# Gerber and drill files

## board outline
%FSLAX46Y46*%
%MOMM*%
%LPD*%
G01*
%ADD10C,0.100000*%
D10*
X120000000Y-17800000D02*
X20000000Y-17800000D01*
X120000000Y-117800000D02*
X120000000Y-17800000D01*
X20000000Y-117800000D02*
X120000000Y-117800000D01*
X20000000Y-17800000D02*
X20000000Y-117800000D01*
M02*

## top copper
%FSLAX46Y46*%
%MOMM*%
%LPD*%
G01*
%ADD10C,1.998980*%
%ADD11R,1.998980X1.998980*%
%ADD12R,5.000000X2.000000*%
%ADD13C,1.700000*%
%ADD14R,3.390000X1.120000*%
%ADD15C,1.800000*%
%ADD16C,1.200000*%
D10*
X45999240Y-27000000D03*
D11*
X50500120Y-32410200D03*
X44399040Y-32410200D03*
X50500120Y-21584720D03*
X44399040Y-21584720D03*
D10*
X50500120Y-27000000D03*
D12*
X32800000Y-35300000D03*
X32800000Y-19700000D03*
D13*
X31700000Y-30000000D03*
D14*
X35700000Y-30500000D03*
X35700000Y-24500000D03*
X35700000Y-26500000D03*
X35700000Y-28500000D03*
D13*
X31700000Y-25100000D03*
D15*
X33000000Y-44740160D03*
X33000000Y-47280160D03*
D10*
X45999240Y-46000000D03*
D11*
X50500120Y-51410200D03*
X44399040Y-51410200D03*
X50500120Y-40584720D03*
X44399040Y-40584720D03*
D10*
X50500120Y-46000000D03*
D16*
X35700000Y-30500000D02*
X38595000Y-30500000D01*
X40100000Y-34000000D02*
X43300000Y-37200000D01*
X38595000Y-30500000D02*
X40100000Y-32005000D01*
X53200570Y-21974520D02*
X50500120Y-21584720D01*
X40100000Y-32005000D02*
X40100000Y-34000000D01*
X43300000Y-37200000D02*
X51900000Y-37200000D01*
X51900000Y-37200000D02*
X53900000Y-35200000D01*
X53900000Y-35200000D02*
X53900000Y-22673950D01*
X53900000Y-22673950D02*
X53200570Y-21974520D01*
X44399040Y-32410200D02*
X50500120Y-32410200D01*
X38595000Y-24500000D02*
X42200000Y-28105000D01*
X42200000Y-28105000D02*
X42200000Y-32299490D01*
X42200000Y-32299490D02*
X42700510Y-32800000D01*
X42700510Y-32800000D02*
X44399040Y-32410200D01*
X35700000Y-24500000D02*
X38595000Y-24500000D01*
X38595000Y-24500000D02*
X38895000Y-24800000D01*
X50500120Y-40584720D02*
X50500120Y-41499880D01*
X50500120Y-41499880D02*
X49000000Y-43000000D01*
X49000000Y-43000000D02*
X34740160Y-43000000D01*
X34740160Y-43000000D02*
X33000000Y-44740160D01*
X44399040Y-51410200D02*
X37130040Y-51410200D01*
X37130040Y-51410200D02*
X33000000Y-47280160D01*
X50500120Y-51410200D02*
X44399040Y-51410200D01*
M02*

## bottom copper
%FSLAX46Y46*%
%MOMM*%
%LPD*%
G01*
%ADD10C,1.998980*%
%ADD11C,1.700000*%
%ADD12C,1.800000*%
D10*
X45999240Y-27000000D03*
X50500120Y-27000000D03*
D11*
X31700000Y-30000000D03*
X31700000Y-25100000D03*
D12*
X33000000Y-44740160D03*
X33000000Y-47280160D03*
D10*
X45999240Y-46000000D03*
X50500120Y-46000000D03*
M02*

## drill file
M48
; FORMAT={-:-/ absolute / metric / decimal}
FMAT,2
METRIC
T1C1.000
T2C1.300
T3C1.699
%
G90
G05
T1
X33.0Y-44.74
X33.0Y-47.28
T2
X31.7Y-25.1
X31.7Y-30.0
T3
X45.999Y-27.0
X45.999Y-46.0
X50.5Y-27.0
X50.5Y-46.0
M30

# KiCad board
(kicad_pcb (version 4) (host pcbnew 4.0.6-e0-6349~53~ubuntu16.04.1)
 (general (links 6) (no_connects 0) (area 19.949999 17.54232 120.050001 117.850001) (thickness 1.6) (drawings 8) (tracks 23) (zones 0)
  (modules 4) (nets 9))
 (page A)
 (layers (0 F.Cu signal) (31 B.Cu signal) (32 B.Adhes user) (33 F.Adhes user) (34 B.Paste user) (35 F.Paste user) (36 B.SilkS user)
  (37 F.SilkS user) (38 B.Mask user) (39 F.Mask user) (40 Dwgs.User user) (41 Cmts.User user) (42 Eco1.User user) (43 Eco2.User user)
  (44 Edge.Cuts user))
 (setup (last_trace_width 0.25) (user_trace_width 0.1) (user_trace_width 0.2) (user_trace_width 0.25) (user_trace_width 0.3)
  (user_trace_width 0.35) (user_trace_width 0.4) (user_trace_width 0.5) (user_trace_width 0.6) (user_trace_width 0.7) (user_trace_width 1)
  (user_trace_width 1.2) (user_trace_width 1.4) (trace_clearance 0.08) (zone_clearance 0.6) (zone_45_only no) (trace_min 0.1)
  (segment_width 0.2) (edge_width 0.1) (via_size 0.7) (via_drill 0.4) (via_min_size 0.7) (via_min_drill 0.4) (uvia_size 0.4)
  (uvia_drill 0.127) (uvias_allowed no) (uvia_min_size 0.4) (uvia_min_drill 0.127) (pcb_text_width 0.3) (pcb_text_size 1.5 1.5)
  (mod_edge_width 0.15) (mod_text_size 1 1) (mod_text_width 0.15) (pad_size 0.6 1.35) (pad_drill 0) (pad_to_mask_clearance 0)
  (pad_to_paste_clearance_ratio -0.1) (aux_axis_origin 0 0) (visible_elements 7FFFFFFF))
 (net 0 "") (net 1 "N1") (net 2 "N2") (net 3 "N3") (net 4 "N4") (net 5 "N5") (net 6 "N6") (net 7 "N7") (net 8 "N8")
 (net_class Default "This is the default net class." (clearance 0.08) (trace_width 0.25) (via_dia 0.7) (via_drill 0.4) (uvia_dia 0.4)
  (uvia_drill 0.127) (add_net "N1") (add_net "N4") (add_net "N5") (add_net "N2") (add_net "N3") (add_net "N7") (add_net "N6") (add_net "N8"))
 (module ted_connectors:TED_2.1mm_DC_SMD (layer F.Cu) (at 47 27)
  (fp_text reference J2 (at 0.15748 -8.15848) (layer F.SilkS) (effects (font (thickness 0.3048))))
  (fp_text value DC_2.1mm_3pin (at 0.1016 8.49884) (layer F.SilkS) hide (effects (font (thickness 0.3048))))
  (pad "" np_thru_hole circle (at -1.00076 0) (size 1.99898 1.99898) (drill 1.69926) (layers *.Cu *.Mask F.SilkS))
  (pad 1 smd rect (at 3.50012 5.4102) (size 1.99898 1.99898) (layers F.Cu F.Paste F.Mask) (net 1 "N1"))
  (pad 1 smd rect (at -2.60096 5.4102) (size 1.99898 1.99898) (layers F.Cu F.Paste F.Mask) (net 1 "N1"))
  (pad 2 smd rect (at 3.50012 -5.41528) (size 1.99898 1.99898) (layers F.Cu F.Paste F.Mask) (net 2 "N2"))
  (pad 3 smd rect (at -2.60096 -5.41528) (size 1.99898 1.99898) (layers F.Cu F.Paste F.Mask) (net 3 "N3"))
  (pad "" np_thru_hole circle (at 3.50012 0) (size 1.99898 1.99898) (drill 1.69926) (layers *.Cu *.Mask F.SilkS)))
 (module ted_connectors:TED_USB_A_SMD (layer F.Cu) (at 28.2 27.5 270)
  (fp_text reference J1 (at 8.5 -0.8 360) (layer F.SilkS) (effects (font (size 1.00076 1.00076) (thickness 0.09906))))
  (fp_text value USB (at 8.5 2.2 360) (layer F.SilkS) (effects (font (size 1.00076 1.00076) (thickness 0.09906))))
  (pad GP smd rect (at 7.8 -4.6 270) (size 2 5) (layers F.Cu F.Paste F.Mask))
  (pad GP smd rect (at -7.8 -4.6 270) (size 2 5) (layers F.Cu F.Paste F.Mask))
  (pad "" np_thru_hole circle (at 2.5 -3.5 270) (size 1.7 1.7) (drill 1.3) (layers *.Cu *.Mask F.SilkS))
  (pad 4 smd rect (at 3 -7.5 270) (size 1.12 3.39) (layers F.Cu F.Paste F.Mask) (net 2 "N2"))
  (pad 1 smd rect (at -3 -7.5 270) (size 1.12 3.39) (layers F.Cu F.Paste F.Mask) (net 1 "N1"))
  (pad 2 smd rect (at -1 -7.5 270) (size 1.12 3.39) (layers F.Cu F.Paste F.Mask) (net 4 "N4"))
  (pad 3 smd rect (at 1 -7.5 270) (size 1.12 3.39) (layers F.Cu F.Paste F.Mask) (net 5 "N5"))
  (pad "" np_thru_hole circle (at -2.4 -3.5 270) (size 1.7 1.7) (drill 1.3) (layers *.Cu *.Mask F.SilkS)))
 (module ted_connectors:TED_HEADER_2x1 (layer F.Cu) (at 33 46 90)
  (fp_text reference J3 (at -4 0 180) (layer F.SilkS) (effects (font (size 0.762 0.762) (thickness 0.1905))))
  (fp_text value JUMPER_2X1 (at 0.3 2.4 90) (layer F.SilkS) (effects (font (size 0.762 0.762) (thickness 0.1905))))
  (pad 2 thru_hole circle (at 1.25984 0 90) (size 1.8 1.8) (drill 1) (layers *.Cu *.Mask F.SilkS) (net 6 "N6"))
  (pad 1 thru_hole circle (at -1.28016 0 90) (size 1.8 1.8) (drill 1) (layers *.Cu *.Mask F.SilkS) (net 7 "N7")))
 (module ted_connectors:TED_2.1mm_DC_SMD (layer F.Cu) (at 47 46)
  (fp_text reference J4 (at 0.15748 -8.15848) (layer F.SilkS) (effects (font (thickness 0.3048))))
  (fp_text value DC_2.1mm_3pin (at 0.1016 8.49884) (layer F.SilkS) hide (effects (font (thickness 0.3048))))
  (pad "" np_thru_hole circle (at -1.00076 0) (size 1.99898 1.99898) (drill 1.69926) (layers *.Cu *.Mask F.SilkS))
  (pad 1 smd rect (at 3.50012 5.4102) (size 1.99898 1.99898) (layers F.Cu F.Paste F.Mask) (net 7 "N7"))
  (pad 1 smd rect (at -2.60096 5.4102) (size 1.99898 1.99898) (layers F.Cu F.Paste F.Mask) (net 7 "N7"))
  (pad 2 smd rect (at 3.50012 -5.41528) (size 1.99898 1.99898) (layers F.Cu F.Paste F.Mask) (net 6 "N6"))
  (pad 3 smd rect (at -2.60096 -5.41528) (size 1.99898 1.99898) (layers F.Cu F.Paste F.Mask) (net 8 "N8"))
  (pad "" np_thru_hole circle (at 3.50012 0) (size 1.99898 1.99898) (drill 1.69926) (layers *.Cu *.Mask F.SilkS)))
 (gr_line (start 120 17.8) (end 20 17.8) (angle 90) (layer Edge.Cuts) (width 0.1))
 (gr_line (start 120 117.8) (end 120 17.8) (angle 90) (layer Edge.Cuts) (width 0.1))
 (gr_line (start 20 117.8) (end 120 117.8) (angle 90) (layer Edge.Cuts) (width 0.1))
 (gr_line (start 20 17.8) (end 20 117.8) (angle 90) (layer Edge.Cuts) (width 0.1))
 (segment (start 35.7 30.5) (end 38.595 30.5) (width 1.2) (layer F.Cu) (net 2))
 (segment (start 40.1 34) (end 43.3 37.2) (width 1.2) (layer F.Cu) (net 2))
 (segment (start 38.595 30.5) (end 40.1 32.005) (width 1.2) (layer F.Cu) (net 2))
 (segment (start 53.20057 21.97452) (end 50.50012 21.58472) (width 1.2) (layer F.Cu) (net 2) (status 20))
 (segment (start 40.1 32.005) (end 40.1 34) (width 1.2) (layer F.Cu) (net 2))
 (segment (start 43.3 37.2) (end 51.9 37.2) (width 1.2) (layer F.Cu) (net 2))
 (segment (start 51.9 37.2) (end 53.9 35.2) (width 1.2) (layer F.Cu) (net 2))
 (segment (start 53.9 35.2) (end 53.9 22.67395) (width 1.2) (layer F.Cu) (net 2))
 (segment (start 53.9 22.67395) (end 53.20057 21.97452) (width 1.2) (layer F.Cu) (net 2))
 (segment (start 44.39904 32.4102) (end 50.50012 32.4102) (width 1.2) (layer F.Cu) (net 1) (status 30))
 (segment (start 38.595 24.5) (end 42.2 28.105) (width 1.2) (layer F.Cu) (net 1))
 (segment (start 42.2 28.105) (end 42.2 32.29949) (width 1.2) (layer F.Cu) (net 1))
 (segment (start 42.2 32.29949) (end 42.70051 32.8) (width 1.2) (layer F.Cu) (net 1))
 (segment (start 42.70051 32.8) (end 44.39904 32.4102) (width 1.2) (layer F.Cu) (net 1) (status 20))
 (segment (start 35.7 24.5) (end 38.595 24.5) (width 1.2) (layer F.Cu) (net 1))
 (segment (start 38.595 24.5) (end 38.895 24.8) (width 1.2) (layer F.Cu) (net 1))
 (segment (start 50.50012 40.58472) (end 50.50012 41.49988) (width 1.2) (layer F.Cu) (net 6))
 (segment (start 50.50012 41.49988) (end 49 43) (width 1.2) (layer F.Cu) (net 6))
 (segment (start 49 43) (end 34.74016 43) (width 1.2) (layer F.Cu) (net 6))
 (segment (start 34.74016 43) (end 33 44.74016) (width 1.2) (layer F.Cu) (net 6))
 (segment (start 44.39904 51.4102) (end 37.13004 51.4102) (width 1.2) (layer F.Cu) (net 7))
 (segment (start 37.13004 51.4102) (end 33 47.28016) (width 1.2) (layer F.Cu) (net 7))
 (segment (start 50.50012 51.4102) (end 44.39904 51.4102) (width 1.2) (layer F.Cu) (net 7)))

